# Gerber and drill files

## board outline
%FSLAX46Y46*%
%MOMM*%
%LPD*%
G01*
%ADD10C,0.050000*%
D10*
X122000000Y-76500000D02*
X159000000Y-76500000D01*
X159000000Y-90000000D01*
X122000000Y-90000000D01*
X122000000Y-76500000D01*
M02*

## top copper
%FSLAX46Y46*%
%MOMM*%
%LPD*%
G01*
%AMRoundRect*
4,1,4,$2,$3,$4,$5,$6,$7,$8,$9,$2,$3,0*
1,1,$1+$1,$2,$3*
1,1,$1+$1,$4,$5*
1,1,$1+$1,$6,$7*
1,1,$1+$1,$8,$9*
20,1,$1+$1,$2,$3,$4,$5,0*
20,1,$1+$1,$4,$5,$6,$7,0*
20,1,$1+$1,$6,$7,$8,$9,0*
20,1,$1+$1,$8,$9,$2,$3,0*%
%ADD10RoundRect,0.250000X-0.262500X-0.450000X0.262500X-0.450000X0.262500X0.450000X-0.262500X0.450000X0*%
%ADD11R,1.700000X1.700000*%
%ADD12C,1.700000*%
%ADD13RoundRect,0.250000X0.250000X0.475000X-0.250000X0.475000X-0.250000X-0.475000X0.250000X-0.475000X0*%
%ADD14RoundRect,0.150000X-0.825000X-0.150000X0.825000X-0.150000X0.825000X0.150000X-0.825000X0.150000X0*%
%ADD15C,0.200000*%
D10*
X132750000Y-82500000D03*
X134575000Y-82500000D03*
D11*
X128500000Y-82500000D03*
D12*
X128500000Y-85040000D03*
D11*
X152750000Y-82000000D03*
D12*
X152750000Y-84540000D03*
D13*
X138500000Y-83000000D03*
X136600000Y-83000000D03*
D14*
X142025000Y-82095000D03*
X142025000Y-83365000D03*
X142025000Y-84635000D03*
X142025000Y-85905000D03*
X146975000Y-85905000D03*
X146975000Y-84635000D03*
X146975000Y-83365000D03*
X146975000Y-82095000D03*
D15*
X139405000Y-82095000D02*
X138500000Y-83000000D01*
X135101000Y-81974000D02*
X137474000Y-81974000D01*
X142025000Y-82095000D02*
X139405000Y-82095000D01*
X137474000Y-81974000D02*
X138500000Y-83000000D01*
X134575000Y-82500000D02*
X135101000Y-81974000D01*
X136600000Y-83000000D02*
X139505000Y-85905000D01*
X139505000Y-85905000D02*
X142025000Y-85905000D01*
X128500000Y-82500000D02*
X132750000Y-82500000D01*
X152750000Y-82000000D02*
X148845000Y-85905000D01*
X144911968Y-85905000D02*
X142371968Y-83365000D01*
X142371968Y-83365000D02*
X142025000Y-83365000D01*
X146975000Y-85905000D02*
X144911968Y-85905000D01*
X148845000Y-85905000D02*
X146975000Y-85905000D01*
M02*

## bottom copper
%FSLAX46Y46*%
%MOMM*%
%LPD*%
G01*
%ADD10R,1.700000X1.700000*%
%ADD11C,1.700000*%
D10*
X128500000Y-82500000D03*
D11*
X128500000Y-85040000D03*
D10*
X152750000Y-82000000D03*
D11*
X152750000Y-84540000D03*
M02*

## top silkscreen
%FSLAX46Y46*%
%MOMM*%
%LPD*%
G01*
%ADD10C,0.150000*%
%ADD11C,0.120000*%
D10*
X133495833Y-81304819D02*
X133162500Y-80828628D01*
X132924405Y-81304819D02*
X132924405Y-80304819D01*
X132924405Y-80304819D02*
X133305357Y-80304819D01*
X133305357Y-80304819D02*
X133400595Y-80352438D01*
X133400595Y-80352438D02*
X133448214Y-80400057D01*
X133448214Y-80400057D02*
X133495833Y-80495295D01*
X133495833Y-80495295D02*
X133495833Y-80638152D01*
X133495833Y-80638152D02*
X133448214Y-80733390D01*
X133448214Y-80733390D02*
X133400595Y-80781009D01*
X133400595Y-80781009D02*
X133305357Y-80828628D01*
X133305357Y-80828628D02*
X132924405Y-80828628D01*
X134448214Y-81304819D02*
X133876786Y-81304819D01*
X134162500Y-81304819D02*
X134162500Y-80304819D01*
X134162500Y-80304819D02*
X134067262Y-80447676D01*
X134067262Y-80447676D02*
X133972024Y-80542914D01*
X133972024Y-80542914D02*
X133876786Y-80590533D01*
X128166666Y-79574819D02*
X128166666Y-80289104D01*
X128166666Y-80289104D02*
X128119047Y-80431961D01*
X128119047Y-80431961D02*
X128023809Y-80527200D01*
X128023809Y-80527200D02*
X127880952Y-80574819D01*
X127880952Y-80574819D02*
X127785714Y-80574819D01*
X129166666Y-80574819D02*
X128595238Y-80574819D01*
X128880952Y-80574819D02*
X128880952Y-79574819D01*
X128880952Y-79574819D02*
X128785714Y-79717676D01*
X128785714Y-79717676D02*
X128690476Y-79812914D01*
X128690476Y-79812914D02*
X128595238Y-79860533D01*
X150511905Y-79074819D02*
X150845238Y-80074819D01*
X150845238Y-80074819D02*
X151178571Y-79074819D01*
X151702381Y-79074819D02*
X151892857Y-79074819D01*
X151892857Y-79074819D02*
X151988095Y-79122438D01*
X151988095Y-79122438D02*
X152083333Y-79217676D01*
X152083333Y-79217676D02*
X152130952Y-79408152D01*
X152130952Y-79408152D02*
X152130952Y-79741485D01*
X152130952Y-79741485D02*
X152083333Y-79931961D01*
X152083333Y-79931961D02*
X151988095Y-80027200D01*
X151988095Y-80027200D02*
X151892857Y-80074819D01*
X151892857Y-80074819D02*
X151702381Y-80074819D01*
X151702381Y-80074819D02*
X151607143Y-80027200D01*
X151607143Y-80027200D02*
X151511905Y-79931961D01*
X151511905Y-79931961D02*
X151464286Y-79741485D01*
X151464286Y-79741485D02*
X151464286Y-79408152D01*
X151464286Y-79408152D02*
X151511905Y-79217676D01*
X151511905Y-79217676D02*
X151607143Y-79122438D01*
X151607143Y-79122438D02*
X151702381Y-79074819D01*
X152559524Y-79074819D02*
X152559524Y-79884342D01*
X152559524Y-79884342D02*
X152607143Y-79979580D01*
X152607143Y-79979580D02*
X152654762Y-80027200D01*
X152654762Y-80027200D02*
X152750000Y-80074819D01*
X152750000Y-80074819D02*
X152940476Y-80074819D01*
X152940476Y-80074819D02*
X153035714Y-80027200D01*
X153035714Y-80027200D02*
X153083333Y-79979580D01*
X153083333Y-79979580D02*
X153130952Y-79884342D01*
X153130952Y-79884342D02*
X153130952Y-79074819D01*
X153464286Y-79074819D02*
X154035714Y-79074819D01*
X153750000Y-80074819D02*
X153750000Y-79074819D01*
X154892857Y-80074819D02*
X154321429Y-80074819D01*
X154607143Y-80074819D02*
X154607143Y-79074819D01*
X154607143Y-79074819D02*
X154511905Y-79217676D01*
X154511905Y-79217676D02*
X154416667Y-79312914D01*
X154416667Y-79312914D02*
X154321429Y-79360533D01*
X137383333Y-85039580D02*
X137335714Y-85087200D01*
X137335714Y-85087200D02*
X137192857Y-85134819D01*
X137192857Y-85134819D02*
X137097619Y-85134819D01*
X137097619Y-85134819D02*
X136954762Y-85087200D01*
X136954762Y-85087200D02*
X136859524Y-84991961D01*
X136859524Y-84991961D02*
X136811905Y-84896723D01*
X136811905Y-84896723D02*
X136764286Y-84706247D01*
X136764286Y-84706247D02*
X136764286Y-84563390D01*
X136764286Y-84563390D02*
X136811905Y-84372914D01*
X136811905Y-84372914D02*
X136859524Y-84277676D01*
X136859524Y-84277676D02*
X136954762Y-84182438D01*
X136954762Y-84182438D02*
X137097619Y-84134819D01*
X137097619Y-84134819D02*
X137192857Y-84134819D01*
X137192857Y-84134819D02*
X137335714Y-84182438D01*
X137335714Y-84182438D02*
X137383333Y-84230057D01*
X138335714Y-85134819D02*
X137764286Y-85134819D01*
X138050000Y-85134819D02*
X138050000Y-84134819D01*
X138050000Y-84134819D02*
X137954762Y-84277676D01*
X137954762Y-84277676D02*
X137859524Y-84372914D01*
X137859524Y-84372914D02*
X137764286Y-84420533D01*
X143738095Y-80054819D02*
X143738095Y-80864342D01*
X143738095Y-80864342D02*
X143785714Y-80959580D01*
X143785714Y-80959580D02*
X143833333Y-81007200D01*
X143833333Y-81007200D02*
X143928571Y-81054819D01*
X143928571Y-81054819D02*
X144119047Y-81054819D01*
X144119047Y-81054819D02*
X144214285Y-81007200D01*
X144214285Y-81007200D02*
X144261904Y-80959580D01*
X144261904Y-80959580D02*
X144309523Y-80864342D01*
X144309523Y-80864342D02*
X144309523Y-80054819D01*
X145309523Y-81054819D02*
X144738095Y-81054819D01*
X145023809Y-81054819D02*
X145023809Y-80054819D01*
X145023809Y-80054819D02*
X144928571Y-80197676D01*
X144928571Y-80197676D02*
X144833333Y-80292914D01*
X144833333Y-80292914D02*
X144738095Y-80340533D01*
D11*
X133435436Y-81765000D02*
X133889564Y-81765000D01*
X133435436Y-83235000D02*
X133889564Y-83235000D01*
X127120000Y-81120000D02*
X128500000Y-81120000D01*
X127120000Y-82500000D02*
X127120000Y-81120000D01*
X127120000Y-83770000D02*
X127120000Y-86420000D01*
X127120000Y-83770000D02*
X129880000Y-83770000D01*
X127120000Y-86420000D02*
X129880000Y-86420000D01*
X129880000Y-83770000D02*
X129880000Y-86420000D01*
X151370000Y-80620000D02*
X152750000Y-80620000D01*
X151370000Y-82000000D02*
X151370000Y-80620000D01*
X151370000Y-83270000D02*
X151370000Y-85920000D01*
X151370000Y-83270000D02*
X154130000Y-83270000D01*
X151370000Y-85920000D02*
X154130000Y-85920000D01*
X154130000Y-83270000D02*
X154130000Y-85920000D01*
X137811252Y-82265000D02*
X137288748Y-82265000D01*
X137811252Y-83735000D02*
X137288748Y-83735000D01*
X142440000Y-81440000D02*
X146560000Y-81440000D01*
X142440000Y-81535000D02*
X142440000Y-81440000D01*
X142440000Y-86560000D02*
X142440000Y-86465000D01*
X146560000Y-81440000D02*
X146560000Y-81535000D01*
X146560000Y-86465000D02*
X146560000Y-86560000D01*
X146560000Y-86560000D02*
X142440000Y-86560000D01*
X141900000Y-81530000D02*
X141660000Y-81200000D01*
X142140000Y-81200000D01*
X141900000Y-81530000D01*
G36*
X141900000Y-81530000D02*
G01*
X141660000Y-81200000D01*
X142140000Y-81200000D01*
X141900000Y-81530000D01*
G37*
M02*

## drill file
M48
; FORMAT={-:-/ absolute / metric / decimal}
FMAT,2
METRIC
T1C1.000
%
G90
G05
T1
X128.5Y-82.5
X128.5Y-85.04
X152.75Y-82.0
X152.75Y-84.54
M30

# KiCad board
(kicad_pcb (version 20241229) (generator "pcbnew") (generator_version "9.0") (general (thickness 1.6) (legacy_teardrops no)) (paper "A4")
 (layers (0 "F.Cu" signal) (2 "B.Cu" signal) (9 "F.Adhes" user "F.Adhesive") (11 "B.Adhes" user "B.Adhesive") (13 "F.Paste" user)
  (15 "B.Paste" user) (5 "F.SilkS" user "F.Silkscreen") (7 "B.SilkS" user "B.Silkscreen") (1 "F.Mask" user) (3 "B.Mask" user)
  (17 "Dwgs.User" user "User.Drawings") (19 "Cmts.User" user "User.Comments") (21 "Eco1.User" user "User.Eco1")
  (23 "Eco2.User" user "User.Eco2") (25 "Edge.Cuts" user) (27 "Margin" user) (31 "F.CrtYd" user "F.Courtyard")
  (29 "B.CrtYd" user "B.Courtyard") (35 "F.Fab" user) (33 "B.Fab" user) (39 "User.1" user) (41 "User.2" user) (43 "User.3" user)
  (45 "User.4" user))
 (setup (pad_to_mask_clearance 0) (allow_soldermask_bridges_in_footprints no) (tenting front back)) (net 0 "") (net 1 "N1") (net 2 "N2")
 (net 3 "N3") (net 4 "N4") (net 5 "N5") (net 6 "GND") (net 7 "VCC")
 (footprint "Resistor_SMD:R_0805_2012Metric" (layer "F.Cu") (at 133.6625 82.5)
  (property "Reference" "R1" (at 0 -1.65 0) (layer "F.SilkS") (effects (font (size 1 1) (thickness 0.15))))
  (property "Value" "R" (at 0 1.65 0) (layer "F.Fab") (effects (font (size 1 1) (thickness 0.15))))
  (fp_line (start -0.227064 -0.735) (end 0.227064 -0.735) (stroke (width 0.12) (type solid)) (layer "F.SilkS"))
  (fp_line (start -0.227064 0.735) (end 0.227064 0.735) (stroke (width 0.12) (type solid)) (layer "F.SilkS"))
  (pad "1" smd roundrect (at -0.9125 0) (size 1.025 1.4) (layers "F.Cu" "F.Mask" "F.Paste") (roundrect_rratio 0.243902) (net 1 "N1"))
  (pad "2" smd roundrect (at 0.9125 0) (size 1.025 1.4) (layers "F.Cu" "F.Mask" "F.Paste") (roundrect_rratio 0.243902) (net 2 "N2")))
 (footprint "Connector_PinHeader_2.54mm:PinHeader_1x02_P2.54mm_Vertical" (layer "F.Cu") (at 128.5 82.5)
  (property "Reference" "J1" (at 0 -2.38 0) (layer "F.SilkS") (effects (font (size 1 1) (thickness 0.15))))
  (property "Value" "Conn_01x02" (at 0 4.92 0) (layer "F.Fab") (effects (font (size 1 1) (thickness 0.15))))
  (fp_line (start -1.38 -1.38) (end 0 -1.38) (stroke (width 0.12) (type solid)) (layer "F.SilkS"))
  (fp_line (start -1.38 0) (end -1.38 -1.38) (stroke (width 0.12) (type solid)) (layer "F.SilkS"))
  (fp_line (start -1.38 1.27) (end -1.38 3.92) (stroke (width 0.12) (type solid)) (layer "F.SilkS"))
  (fp_line (start -1.38 1.27) (end 1.38 1.27) (stroke (width 0.12) (type solid)) (layer "F.SilkS"))
  (fp_line (start -1.38 3.92) (end 1.38 3.92) (stroke (width 0.12) (type solid)) (layer "F.SilkS"))
  (fp_line (start 1.38 1.27) (end 1.38 3.92) (stroke (width 0.12) (type solid)) (layer "F.SilkS"))
  (pad "1" thru_hole rect (at 0 0) (size 1.7 1.7) (drill 1) (layers "*.Cu" "*.Mask") (remove_unused_layers no) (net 1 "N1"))
  (pad "2" thru_hole circle (at 0 2.54) (size 1.7 1.7) (drill 1) (layers "*.Cu" "*.Mask") (remove_unused_layers no) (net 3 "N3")))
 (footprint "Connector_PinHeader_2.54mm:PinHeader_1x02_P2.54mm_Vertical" (layer "F.Cu") (at 152.75 82)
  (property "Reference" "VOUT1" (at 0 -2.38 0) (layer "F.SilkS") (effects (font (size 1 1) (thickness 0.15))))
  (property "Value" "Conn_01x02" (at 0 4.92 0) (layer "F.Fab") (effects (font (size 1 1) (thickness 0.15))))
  (fp_line (start -1.38 -1.38) (end 0 -1.38) (stroke (width 0.12) (type solid)) (layer "F.SilkS"))
  (fp_line (start -1.38 0) (end -1.38 -1.38) (stroke (width 0.12) (type solid)) (layer "F.SilkS"))
  (fp_line (start -1.38 1.27) (end -1.38 3.92) (stroke (width 0.12) (type solid)) (layer "F.SilkS"))
  (fp_line (start -1.38 1.27) (end 1.38 1.27) (stroke (width 0.12) (type solid)) (layer "F.SilkS"))
  (fp_line (start -1.38 3.92) (end 1.38 3.92) (stroke (width 0.12) (type solid)) (layer "F.SilkS"))
  (fp_line (start 1.38 1.27) (end 1.38 3.92) (stroke (width 0.12) (type solid)) (layer "F.SilkS"))
  (pad "1" thru_hole rect (at 0 0) (size 1.7 1.7) (drill 1) (layers "*.Cu" "*.Mask") (remove_unused_layers no) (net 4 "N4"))
  (pad "2" thru_hole circle (at 0 2.54) (size 1.7 1.7) (drill 1) (layers "*.Cu" "*.Mask") (remove_unused_layers no) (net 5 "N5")))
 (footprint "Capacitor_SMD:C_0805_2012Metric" (layer "F.Cu") (at 137.55 83 180)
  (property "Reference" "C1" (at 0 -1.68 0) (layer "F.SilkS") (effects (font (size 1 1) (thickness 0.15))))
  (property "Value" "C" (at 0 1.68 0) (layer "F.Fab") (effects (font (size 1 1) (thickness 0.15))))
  (fp_line (start -0.261252 0.735) (end 0.261252 0.735) (stroke (width 0.12) (type solid)) (layer "F.SilkS"))
  (fp_line (start -0.261252 -0.735) (end 0.261252 -0.735) (stroke (width 0.12) (type solid)) (layer "F.SilkS"))
  (pad "1" smd roundrect (at -0.95 0 180) (size 1 1.45) (layers "F.Cu" "F.Mask" "F.Paste") (roundrect_rratio 0.25) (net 2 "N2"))
  (pad "2" smd roundrect (at 0.95 0 180) (size 1 1.45) (layers "F.Cu" "F.Mask" "F.Paste") (roundrect_rratio 0.25) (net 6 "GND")))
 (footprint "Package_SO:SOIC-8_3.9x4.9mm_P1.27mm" (layer "F.Cu") (at 144.5 84)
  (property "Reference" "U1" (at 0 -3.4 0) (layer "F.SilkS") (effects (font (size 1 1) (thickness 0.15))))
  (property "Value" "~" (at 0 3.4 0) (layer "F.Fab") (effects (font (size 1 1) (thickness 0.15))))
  (fp_line (start -2.06 -2.56) (end 2.06 -2.56) (stroke (width 0.12) (type solid)) (layer "F.SilkS"))
  (fp_line (start -2.06 -2.465) (end -2.06 -2.56) (stroke (width 0.12) (type solid)) (layer "F.SilkS"))
  (fp_line (start -2.06 2.56) (end -2.06 2.465) (stroke (width 0.12) (type solid)) (layer "F.SilkS"))
  (fp_line (start 2.06 -2.56) (end 2.06 -2.465) (stroke (width 0.12) (type solid)) (layer "F.SilkS"))
  (fp_line (start 2.06 2.465) (end 2.06 2.56) (stroke (width 0.12) (type solid)) (layer "F.SilkS"))
  (fp_line (start 2.06 2.56) (end -2.06 2.56) (stroke (width 0.12) (type solid)) (layer "F.SilkS"))
  (fp_poly (pts (xy -2.6 -2.47) (xy -2.84 -2.8) (xy -2.36 -2.8)) (stroke (width 0.12) (type solid)) (fill yes) (layer "F.SilkS"))
  (pad "1" smd roundrect (at -2.475 -1.905) (size 1.95 0.6) (layers "F.Cu" "F.Mask" "F.Paste") (roundrect_rratio 0.25) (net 2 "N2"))
  (pad "2" smd roundrect (at -2.475 -0.635) (size 1.95 0.6) (layers "F.Cu" "F.Mask" "F.Paste") (roundrect_rratio 0.25) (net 4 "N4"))
  (pad "3" smd roundrect (at -2.475 0.635) (size 1.95 0.6) (layers "F.Cu" "F.Mask" "F.Paste") (roundrect_rratio 0.25) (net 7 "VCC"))
  (pad "4" smd roundrect (at -2.475 1.905) (size 1.95 0.6) (layers "F.Cu" "F.Mask" "F.Paste") (roundrect_rratio 0.25) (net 6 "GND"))
  (pad "5" smd roundrect (at 2.475 1.905) (size 1.95 0.6) (layers "F.Cu" "F.Mask" "F.Paste") (roundrect_rratio 0.25) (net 4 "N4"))
  (pad "6" smd roundrect (at 2.475 0.635) (size 1.95 0.6) (layers "F.Cu" "F.Mask" "F.Paste") (roundrect_rratio 0.25))
  (pad "7" smd roundrect (at 2.475 -0.635) (size 1.95 0.6) (layers "F.Cu" "F.Mask" "F.Paste") (roundrect_rratio 0.25))
  (pad "8" smd roundrect (at 2.475 -1.905) (size 1.95 0.6) (layers "F.Cu" "F.Mask" "F.Paste") (roundrect_rratio 0.25)))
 (gr_rect (start 122 76.5) (end 159 90) (stroke (width 0.05) (type default)) (fill no) (layer "Edge.Cuts"))
 (segment (start 139.405 82.095) (end 138.5 83) (width 0.2) (layer "F.Cu") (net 2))
 (segment (start 135.101 81.974) (end 137.474 81.974) (width 0.2) (layer "F.Cu") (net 2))
 (segment (start 142.025 82.095) (end 139.405 82.095) (width 0.2) (layer "F.Cu") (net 2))
 (segment (start 137.474 81.974) (end 138.5 83) (width 0.2) (layer "F.Cu") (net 2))
 (segment (start 134.575 82.5) (end 135.101 81.974) (width 0.2) (layer "F.Cu") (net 2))
 (segment (start 136.6 83) (end 139.505 85.905) (width 0.2) (layer "F.Cu") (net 6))
 (segment (start 139.505 85.905) (end 142.025 85.905) (width 0.2) (layer "F.Cu") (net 6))
 (segment (start 128.5 82.5) (end 132.75 82.5) (width 0.2) (layer "F.Cu") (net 1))
 (segment (start 152.75 82) (end 148.845 85.905) (width 0.2) (layer "F.Cu") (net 4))
 (segment (start 144.911968 85.905) (end 142.371968 83.365) (width 0.2) (layer "F.Cu") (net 4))
 (segment (start 142.371968 83.365) (end 142.025 83.365) (width 0.2) (layer "F.Cu") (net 4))
 (segment (start 146.975 85.905) (end 144.911968 85.905) (width 0.2) (layer "F.Cu") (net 4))
 (segment (start 148.845 85.905) (end 146.975 85.905) (width 0.2) (layer "F.Cu") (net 4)))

